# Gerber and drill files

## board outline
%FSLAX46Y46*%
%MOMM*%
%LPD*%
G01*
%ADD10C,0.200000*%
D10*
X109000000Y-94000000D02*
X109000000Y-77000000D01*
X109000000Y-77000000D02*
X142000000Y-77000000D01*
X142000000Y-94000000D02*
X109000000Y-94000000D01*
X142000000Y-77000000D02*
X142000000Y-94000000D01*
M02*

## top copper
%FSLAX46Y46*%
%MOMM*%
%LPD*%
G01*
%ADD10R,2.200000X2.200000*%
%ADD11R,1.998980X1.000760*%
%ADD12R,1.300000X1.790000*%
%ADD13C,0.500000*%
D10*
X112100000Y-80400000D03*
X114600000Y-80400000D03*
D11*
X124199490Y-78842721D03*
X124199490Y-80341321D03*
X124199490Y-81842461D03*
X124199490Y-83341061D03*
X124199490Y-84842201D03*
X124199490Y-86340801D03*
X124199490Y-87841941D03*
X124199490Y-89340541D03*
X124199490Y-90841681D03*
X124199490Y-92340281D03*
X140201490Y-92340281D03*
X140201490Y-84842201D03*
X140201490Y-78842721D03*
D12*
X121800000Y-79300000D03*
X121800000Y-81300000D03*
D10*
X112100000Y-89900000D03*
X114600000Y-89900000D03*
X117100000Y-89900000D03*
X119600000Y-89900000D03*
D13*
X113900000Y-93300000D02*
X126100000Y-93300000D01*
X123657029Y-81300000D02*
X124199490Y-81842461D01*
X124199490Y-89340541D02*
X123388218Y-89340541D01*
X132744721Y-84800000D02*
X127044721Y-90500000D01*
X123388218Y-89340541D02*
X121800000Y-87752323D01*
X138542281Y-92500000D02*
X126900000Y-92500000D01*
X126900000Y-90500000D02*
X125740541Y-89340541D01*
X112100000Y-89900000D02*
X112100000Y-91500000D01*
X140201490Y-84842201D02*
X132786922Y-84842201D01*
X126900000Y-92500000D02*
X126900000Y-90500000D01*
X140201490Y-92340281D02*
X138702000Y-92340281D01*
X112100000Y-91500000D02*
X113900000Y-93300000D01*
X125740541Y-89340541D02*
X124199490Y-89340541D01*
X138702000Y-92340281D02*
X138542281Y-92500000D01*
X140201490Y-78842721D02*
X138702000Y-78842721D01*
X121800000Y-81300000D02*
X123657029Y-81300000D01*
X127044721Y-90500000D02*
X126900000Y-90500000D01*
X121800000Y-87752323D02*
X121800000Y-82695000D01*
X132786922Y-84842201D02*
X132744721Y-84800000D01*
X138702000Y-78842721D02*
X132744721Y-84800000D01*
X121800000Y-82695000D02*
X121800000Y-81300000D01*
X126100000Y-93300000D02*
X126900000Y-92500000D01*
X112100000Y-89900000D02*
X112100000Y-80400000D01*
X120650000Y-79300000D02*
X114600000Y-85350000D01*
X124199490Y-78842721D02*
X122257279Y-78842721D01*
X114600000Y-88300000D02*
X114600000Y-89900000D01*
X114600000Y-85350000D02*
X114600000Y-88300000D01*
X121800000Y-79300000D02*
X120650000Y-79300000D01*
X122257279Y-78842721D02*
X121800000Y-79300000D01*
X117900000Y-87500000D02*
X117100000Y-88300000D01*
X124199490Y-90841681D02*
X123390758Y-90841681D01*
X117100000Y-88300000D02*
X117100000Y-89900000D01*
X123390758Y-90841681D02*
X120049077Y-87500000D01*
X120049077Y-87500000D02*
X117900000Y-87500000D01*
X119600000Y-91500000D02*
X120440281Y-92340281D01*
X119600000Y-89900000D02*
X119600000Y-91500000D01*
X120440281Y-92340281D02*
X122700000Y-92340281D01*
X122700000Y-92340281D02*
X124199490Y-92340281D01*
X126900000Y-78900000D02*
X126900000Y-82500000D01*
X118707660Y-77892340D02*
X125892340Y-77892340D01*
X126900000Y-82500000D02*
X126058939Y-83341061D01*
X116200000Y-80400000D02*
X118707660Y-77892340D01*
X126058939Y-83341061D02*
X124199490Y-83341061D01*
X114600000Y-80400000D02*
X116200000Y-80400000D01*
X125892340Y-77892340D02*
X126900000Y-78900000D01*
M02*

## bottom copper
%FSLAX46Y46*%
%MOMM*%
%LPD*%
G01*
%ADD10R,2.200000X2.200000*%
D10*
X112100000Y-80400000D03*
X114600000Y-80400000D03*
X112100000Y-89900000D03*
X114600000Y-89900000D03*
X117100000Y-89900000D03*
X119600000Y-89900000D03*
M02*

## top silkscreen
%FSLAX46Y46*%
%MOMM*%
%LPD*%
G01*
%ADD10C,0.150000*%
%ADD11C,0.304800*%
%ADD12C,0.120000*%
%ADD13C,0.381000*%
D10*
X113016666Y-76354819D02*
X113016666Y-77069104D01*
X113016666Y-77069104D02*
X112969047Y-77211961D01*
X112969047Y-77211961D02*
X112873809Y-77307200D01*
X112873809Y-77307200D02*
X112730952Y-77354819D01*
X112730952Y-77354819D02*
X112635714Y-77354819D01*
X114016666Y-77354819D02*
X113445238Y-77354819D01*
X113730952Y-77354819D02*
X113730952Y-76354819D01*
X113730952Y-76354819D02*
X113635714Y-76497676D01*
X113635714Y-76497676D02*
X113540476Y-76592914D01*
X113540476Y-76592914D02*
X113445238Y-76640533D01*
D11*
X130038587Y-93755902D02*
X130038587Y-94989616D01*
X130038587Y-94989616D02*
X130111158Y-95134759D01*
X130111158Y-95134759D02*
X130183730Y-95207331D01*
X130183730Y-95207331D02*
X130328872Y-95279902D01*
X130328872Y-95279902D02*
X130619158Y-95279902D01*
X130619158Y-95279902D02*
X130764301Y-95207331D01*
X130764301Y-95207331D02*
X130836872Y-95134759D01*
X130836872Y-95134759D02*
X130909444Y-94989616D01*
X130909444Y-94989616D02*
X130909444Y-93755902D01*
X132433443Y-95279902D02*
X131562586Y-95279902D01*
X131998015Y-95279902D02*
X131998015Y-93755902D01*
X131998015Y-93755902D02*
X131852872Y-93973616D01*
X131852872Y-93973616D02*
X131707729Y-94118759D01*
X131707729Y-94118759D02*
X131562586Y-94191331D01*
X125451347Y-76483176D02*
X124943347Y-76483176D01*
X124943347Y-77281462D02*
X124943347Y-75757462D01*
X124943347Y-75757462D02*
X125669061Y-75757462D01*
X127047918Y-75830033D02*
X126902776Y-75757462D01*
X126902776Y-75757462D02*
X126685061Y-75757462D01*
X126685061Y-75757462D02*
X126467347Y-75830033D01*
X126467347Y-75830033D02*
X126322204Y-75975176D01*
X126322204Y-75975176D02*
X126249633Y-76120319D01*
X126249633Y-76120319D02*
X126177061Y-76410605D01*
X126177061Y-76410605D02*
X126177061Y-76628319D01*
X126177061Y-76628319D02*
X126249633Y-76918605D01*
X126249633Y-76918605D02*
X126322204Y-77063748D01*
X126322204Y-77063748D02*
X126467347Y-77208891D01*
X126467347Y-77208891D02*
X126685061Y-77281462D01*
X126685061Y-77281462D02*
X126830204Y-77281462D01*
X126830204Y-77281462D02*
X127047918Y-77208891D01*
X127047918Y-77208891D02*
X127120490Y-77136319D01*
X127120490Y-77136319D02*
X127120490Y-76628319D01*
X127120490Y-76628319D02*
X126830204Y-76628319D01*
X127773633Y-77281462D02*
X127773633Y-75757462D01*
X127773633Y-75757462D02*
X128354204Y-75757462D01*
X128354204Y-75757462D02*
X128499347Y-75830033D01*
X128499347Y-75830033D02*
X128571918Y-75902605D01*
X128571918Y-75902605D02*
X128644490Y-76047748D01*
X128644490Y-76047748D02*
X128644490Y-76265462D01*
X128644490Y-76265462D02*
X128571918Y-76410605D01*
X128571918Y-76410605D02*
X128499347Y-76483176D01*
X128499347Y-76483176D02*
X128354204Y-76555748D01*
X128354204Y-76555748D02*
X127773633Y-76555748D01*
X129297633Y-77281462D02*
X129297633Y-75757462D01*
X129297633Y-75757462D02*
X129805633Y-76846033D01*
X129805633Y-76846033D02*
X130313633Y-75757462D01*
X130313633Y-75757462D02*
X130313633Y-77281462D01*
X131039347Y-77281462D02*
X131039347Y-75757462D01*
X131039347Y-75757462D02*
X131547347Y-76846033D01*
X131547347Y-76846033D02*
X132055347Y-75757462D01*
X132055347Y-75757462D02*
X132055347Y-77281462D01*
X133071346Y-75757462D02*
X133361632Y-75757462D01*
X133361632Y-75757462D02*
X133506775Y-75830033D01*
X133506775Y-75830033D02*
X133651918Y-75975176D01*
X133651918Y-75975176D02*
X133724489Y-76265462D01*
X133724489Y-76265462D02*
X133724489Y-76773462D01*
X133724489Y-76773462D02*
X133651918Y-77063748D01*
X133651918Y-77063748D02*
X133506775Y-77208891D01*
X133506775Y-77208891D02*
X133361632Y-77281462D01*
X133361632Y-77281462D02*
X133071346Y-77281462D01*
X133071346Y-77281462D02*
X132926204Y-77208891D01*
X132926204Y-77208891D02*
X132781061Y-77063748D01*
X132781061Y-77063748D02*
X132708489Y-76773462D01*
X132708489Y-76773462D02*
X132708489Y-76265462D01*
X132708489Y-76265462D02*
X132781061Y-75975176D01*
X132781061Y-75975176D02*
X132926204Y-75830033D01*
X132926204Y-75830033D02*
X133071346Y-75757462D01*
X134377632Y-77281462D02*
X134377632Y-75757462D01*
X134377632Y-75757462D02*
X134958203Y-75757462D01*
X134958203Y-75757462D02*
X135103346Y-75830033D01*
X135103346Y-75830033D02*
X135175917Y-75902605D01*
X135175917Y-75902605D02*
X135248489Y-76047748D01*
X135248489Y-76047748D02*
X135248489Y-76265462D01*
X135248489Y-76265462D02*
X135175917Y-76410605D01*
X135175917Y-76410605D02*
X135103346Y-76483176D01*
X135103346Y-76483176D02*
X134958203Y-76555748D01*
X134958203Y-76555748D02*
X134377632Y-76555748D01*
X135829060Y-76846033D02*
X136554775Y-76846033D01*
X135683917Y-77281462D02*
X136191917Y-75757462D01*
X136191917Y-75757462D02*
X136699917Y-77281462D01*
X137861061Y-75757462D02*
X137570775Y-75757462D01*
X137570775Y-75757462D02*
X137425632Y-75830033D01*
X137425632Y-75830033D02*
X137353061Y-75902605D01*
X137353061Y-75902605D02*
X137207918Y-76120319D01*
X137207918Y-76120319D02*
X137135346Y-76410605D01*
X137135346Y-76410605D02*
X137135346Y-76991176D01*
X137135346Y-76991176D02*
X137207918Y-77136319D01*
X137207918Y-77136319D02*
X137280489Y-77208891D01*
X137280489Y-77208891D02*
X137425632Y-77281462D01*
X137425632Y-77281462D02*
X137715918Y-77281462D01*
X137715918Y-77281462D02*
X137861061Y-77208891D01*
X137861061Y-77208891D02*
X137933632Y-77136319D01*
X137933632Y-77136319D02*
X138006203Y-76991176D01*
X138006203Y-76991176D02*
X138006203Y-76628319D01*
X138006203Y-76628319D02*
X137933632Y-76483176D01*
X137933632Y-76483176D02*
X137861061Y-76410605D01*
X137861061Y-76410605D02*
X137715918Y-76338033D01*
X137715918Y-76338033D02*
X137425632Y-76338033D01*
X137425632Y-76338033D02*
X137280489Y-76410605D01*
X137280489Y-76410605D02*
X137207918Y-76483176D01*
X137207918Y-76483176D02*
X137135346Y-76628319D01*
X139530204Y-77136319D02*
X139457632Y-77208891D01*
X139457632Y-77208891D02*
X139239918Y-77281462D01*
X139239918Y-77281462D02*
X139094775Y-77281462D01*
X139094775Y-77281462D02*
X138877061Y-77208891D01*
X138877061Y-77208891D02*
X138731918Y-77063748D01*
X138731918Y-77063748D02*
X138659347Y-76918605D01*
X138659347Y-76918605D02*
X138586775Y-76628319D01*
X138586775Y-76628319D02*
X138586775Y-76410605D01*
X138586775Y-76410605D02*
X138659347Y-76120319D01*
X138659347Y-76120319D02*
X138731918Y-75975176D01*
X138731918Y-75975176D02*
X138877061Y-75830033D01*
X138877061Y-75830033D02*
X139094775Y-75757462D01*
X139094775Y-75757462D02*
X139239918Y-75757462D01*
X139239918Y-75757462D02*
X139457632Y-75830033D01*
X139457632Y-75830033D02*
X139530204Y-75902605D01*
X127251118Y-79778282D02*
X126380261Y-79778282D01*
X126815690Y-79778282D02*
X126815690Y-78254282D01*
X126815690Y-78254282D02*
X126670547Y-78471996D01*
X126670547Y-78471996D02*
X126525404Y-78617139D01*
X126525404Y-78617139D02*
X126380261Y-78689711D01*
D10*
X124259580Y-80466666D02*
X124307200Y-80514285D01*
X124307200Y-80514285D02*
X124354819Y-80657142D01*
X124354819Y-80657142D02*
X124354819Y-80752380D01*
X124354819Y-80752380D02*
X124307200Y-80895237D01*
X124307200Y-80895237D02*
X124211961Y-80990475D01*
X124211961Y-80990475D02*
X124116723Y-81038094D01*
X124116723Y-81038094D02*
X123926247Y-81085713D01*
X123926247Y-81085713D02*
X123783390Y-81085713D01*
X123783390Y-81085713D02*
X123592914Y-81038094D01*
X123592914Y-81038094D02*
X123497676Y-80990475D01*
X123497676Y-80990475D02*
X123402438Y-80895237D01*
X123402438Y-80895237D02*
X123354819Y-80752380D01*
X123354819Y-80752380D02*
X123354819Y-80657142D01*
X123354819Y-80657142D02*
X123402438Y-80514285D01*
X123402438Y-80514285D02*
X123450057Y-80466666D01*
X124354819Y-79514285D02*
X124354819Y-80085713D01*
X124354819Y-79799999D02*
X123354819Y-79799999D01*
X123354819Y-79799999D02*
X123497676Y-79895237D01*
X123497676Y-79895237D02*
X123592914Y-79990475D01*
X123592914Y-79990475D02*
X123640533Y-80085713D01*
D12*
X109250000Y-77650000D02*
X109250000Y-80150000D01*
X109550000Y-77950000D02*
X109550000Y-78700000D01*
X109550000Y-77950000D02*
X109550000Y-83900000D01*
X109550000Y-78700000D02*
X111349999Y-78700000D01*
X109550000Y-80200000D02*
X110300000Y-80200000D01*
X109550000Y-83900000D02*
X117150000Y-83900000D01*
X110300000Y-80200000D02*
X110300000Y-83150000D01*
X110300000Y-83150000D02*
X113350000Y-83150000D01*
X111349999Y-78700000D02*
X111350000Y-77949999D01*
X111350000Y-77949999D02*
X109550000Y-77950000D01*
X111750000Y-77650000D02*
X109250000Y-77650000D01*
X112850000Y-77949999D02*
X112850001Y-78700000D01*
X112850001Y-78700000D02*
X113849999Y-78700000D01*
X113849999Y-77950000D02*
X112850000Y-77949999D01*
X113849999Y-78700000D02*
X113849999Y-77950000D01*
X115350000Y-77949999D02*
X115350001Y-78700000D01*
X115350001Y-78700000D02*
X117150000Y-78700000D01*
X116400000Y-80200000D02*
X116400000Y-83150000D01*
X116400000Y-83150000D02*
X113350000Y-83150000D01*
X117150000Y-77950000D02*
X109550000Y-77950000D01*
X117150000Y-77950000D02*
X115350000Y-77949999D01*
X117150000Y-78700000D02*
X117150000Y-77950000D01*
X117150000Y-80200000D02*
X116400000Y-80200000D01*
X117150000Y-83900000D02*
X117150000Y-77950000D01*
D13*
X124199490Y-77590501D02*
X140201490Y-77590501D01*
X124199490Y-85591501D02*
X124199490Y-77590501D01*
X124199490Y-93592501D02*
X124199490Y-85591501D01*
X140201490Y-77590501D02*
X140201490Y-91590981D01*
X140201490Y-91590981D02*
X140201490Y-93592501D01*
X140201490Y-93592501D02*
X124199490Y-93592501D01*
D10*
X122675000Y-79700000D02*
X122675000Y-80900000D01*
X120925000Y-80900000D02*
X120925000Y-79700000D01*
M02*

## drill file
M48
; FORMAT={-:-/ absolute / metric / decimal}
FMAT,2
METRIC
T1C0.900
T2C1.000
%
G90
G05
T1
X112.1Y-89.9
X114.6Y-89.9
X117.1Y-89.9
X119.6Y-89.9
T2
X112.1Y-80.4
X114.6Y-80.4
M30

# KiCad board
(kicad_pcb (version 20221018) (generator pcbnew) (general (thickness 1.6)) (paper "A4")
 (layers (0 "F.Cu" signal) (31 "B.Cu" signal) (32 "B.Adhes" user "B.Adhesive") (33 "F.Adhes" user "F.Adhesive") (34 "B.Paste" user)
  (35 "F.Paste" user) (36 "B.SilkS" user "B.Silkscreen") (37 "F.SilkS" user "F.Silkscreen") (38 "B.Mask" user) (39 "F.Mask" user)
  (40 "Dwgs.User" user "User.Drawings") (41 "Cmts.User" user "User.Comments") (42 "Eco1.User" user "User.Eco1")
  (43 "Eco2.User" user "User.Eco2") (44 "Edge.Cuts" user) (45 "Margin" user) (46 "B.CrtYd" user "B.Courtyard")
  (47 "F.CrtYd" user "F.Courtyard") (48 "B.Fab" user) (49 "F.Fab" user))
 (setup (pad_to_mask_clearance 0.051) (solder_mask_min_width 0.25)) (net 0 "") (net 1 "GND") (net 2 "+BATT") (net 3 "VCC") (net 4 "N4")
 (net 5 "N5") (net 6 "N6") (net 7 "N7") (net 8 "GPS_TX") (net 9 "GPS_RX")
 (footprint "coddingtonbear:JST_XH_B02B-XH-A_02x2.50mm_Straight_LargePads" (layer "F.Cu") (at 112.1 80.4)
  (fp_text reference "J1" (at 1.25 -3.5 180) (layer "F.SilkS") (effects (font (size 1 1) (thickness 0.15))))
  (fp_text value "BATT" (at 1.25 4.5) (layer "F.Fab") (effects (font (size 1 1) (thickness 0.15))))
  (fp_line (start -2.85 -2.75) (end -2.85 -0.25) (stroke (width 0.12) (type solid)) (layer "F.SilkS"))
  (fp_line (start -2.55 -2.45) (end -2.55 -1.7) (stroke (width 0.12) (type solid)) (layer "F.SilkS"))
  (fp_line (start -2.55 -2.45) (end -2.55 3.5) (stroke (width 0.12) (type solid)) (layer "F.SilkS"))
  (fp_line (start -2.55 -1.7) (end -0.750001 -1.7) (stroke (width 0.12) (type solid)) (layer "F.SilkS"))
  (fp_line (start -2.55 -0.2) (end -1.8 -0.2) (stroke (width 0.12) (type solid)) (layer "F.SilkS"))
  (fp_line (start -2.55 3.5) (end 5.05 3.5) (stroke (width 0.12) (type solid)) (layer "F.SilkS"))
  (fp_line (start -1.8 -0.2) (end -1.8 2.75) (stroke (width 0.12) (type solid)) (layer "F.SilkS"))
  (fp_line (start -1.8 2.75) (end 1.25 2.75) (stroke (width 0.12) (type solid)) (layer "F.SilkS"))
  (fp_line (start -0.750001 -1.7) (end -0.75 -2.450001) (stroke (width 0.12) (type solid)) (layer "F.SilkS"))
  (fp_line (start -0.75 -2.450001) (end -2.55 -2.45) (stroke (width 0.12) (type solid)) (layer "F.SilkS"))
  (fp_line (start -0.35 -2.75) (end -2.85 -2.75) (stroke (width 0.12) (type solid)) (layer "F.SilkS"))
  (fp_line (start 0.75 -2.450001) (end 0.750001 -1.7) (stroke (width 0.12) (type solid)) (layer "F.SilkS"))
  (fp_line (start 0.750001 -1.7) (end 1.749999 -1.7) (stroke (width 0.12) (type solid)) (layer "F.SilkS"))
  (fp_line (start 1.749999 -2.45) (end 0.75 -2.450001) (stroke (width 0.12) (type solid)) (layer "F.SilkS"))
  (fp_line (start 1.749999 -1.7) (end 1.749999 -2.45) (stroke (width 0.12) (type solid)) (layer "F.SilkS"))
  (fp_line (start 3.25 -2.450001) (end 3.250001 -1.7) (stroke (width 0.12) (type solid)) (layer "F.SilkS"))
  (fp_line (start 3.250001 -1.7) (end 5.05 -1.7) (stroke (width 0.12) (type solid)) (layer "F.SilkS"))
  (fp_line (start 4.3 -0.2) (end 4.3 2.75) (stroke (width 0.12) (type solid)) (layer "F.SilkS"))
  (fp_line (start 4.3 2.75) (end 1.25 2.75) (stroke (width 0.12) (type solid)) (layer "F.SilkS"))
  (fp_line (start 5.05 -2.45) (end -2.55 -2.45) (stroke (width 0.12) (type solid)) (layer "F.SilkS"))
  (fp_line (start 5.05 -2.45) (end 3.25 -2.450001) (stroke (width 0.12) (type solid)) (layer "F.SilkS"))
  (fp_line (start 5.05 -1.7) (end 5.05 -2.45) (stroke (width 0.12) (type solid)) (layer "F.SilkS"))
  (fp_line (start 5.05 -0.2) (end 4.3 -0.2) (stroke (width 0.12) (type solid)) (layer "F.SilkS"))
  (fp_line (start 5.05 3.5) (end 5.05 -2.45) (stroke (width 0.12) (type solid)) (layer "F.SilkS"))
  (pad "1" thru_hole rect (at 0 0) (size 2.2 2.2) (drill 1) (layers "*.Cu" "*.Mask") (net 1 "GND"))
  (pad "2" thru_hole rect (at 2.5 0) (size 2.2 2.2) (drill 1) (layers "*.Cu" "*.Mask") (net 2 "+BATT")))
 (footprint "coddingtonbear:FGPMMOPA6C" (layer "F.Cu") (at 132.20049 85.591501)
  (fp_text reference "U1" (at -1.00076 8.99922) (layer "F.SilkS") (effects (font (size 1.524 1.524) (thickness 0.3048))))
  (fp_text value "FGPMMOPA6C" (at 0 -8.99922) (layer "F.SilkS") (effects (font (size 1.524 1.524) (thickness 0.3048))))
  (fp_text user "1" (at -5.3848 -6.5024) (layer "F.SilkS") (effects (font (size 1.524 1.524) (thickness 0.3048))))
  (fp_line (start -8.001 -8.001) (end 8.001 -8.001) (stroke (width 0.381) (type solid)) (layer "F.SilkS"))
  (fp_line (start -8.001 0) (end -8.001 -8.001) (stroke (width 0.381) (type solid)) (layer "F.SilkS"))
  (fp_line (start -8.001 8.001) (end -8.001 0) (stroke (width 0.381) (type solid)) (layer "F.SilkS"))
  (fp_line (start 8.001 -8.001) (end 8.001 5.99948) (stroke (width 0.381) (type solid)) (layer "F.SilkS"))
  (fp_line (start 8.001 5.99948) (end 8.001 8.001) (stroke (width 0.381) (type solid)) (layer "F.SilkS"))
  (fp_line (start 8.001 8.001) (end -8.001 8.001) (stroke (width 0.381) (type solid)) (layer "F.SilkS"))
  (pad "1" smd rect (at -8.001 -6.74878) (size 1.99898 1.00076) (layers "F.Cu" "F.Paste" "F.Mask") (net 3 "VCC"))
  (pad "2" smd rect (at -8.001 -5.25018) (size 1.99898 1.00076) (layers "F.Cu" "F.Paste" "F.Mask") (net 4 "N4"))
  (pad "3" smd rect (at -8.001 -3.74904) (size 1.99898 1.00076) (layers "F.Cu" "F.Paste" "F.Mask") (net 1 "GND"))
  (pad "4" smd rect (at -8.001 -2.25044) (size 1.99898 1.00076) (layers "F.Cu" "F.Paste" "F.Mask") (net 2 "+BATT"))
  (pad "5" smd rect (at -8.001 -0.7493) (size 1.99898 1.00076) (layers "F.Cu" "F.Paste" "F.Mask") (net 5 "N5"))
  (pad "6" smd rect (at -8.001 0.7493) (size 1.99898 1.00076) (layers "F.Cu" "F.Paste" "F.Mask") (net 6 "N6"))
  (pad "7" smd rect (at -8.001 2.25044) (size 1.99898 1.00076) (layers "F.Cu" "F.Paste" "F.Mask") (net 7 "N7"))
  (pad "8" smd rect (at -8.001 3.74904) (size 1.99898 1.00076) (layers "F.Cu" "F.Paste" "F.Mask") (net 1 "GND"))
  (pad "9" smd rect (at -8.001 5.25018) (size 1.99898 1.00076) (layers "F.Cu" "F.Paste" "F.Mask") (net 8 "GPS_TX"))
  (pad "10" smd rect (at -8.001 6.74878) (size 1.99898 1.00076) (layers "F.Cu" "F.Paste" "F.Mask") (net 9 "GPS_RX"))
  (pad "11" smd rect (at 8.001 6.74878) (size 1.99898 1.00076) (layers "F.Cu" "F.Paste" "F.Mask") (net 1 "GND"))
  (pad "12" smd rect (at 8.001 -0.7493) (size 1.99898 1.00076) (layers "F.Cu" "F.Paste" "F.Mask") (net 1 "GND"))
  (pad "13" smd rect (at 8.001 -6.74878) (size 1.99898 1.00076) (layers "F.Cu" "F.Paste" "F.Mask") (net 1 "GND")))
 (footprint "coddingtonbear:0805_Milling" (layer "F.Cu") (at 121.8 80.3 -90)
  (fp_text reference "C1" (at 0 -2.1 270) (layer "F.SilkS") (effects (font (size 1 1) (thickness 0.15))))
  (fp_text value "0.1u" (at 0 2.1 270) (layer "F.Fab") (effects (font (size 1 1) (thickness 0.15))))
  (fp_line (start -0.6 -0.875) (end 0.6 -0.875) (stroke (width 0.15) (type solid)) (layer "F.SilkS"))
  (fp_line (start 0.6 0.875) (end -0.6 0.875) (stroke (width 0.15) (type solid)) (layer "F.SilkS"))
  (pad "1" smd rect (at -1 0 270) (size 1.79 1.3) (layers "F.Cu" "F.Paste" "F.Mask") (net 3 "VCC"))
  (pad "2" smd rect (at 1 0 270) (size 1.79 1.3) (layers "F.Cu" "F.Paste" "F.Mask") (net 1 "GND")))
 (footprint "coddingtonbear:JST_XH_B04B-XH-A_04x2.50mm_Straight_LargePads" (layer "B.Cu") (at 112.1 89.9)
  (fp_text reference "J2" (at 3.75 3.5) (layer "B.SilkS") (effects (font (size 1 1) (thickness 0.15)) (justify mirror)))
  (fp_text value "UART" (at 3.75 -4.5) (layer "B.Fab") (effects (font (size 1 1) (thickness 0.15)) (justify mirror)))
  (pad "1" thru_hole rect (at 0 0) (size 2.2 2.2) (drill 0.9) (layers "*.Cu" "*.Mask") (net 1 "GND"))
  (pad "2" thru_hole rect (at 2.5 0) (size 2.2 2.2) (drill 0.9) (layers "*.Cu" "*.Mask") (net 3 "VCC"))
  (pad "3" thru_hole rect (at 5 0) (size 2.2 2.2) (drill 0.9) (layers "*.Cu" "*.Mask") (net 8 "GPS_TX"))
  (pad "4" thru_hole rect (at 7.5 0) (size 2.2 2.2) (drill 0.9) (layers "*.Cu" "*.Mask") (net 9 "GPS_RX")))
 (gr_line (start 109 94) (end 109 77) (stroke (width 0.2) (type solid)) (layer "Edge.Cuts"))
 (gr_line (start 109 77) (end 142 77) (stroke (width 0.2) (type solid)) (layer "Edge.Cuts"))
 (gr_line (start 142 94) (end 109 94) (stroke (width 0.2) (type solid)) (layer "Edge.Cuts"))
 (gr_line (start 142 77) (end 142 94) (stroke (width 0.2) (type solid)) (layer "Edge.Cuts"))
 (segment (start 113.9 93.3) (end 126.1 93.3) (width 0.5) (layer "F.Cu") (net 1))
 (segment (start 123.657029 81.3) (end 124.19949 81.842461) (width 0.5) (layer "F.Cu") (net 1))
 (segment (start 124.19949 89.340541) (end 123.388218 89.340541) (width 0.5) (layer "F.Cu") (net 1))
 (segment (start 132.744721 84.8) (end 127.044721 90.5) (width 0.5) (layer "F.Cu") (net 1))
 (segment (start 123.388218 89.340541) (end 121.8 87.752323) (width 0.5) (layer "F.Cu") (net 1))
 (segment (start 138.542281 92.5) (end 126.9 92.5) (width 0.5) (layer "F.Cu") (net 1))
 (segment (start 126.9 90.5) (end 125.740541 89.340541) (width 0.5) (layer "F.Cu") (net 1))
 (segment (start 112.1 89.9) (end 112.1 91.5) (width 0.5) (layer "F.Cu") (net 1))
 (segment (start 140.20149 84.842201) (end 132.786922 84.842201) (width 0.5) (layer "F.Cu") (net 1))
 (segment (start 126.9 92.5) (end 126.9 90.5) (width 0.5) (layer "F.Cu") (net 1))
 (segment (start 140.20149 92.340281) (end 138.702 92.340281) (width 0.5) (layer "F.Cu") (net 1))
 (segment (start 112.1 91.5) (end 113.9 93.3) (width 0.5) (layer "F.Cu") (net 1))
 (segment (start 125.740541 89.340541) (end 124.19949 89.340541) (width 0.5) (layer "F.Cu") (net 1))
 (segment (start 138.702 92.340281) (end 138.542281 92.5) (width 0.5) (layer "F.Cu") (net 1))
 (segment (start 140.20149 78.842721) (end 138.702 78.842721) (width 0.5) (layer "F.Cu") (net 1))
 (segment (start 121.8 81.3) (end 123.657029 81.3) (width 0.5) (layer "F.Cu") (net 1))
 (segment (start 127.044721 90.5) (end 126.9 90.5) (width 0.5) (layer "F.Cu") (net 1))
 (segment (start 121.8 87.752323) (end 121.8 82.695) (width 0.5) (layer "F.Cu") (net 1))
 (segment (start 132.786922 84.842201) (end 132.744721 84.8) (width 0.5) (layer "F.Cu") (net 1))
 (segment (start 138.702 78.842721) (end 132.744721 84.8) (width 0.5) (layer "F.Cu") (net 1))
 (segment (start 121.8 82.695) (end 121.8 81.3) (width 0.5) (layer "F.Cu") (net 1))
 (segment (start 126.1 93.3) (end 126.9 92.5) (width 0.5) (layer "F.Cu") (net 1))
 (segment (start 112.1 89.9) (end 112.1 80.4) (width 0.5) (layer "F.Cu") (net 1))
 (segment (start 120.65 79.3) (end 114.6 85.35) (width 0.5) (layer "F.Cu") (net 3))
 (segment (start 124.19949 78.842721) (end 122.257279 78.842721) (width 0.5) (layer "F.Cu") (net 3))
 (segment (start 114.6 88.3) (end 114.6 89.9) (width 0.5) (layer "F.Cu") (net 3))
 (segment (start 114.6 85.35) (end 114.6 88.3) (width 0.5) (layer "F.Cu") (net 3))
 (segment (start 121.8 79.3) (end 120.65 79.3) (width 0.5) (layer "F.Cu") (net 3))
 (segment (start 122.257279 78.842721) (end 121.8 79.3) (width 0.5) (layer "F.Cu") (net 3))
 (segment (start 117.9 87.5) (end 117.1 88.3) (width 0.5) (layer "F.Cu") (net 8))
 (segment (start 124.19949 90.841681) (end 123.390758 90.841681) (width 0.5) (layer "F.Cu") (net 8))
 (segment (start 117.1 88.3) (end 117.1 89.9) (width 0.5) (layer "F.Cu") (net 8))
 (segment (start 123.390758 90.841681) (end 120.049077 87.5) (width 0.5) (layer "F.Cu") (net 8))
 (segment (start 120.049077 87.5) (end 117.9 87.5) (width 0.5) (layer "F.Cu") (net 8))
 (segment (start 119.6 91.5) (end 120.440281 92.340281) (width 0.5) (layer "F.Cu") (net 9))
 (segment (start 119.6 89.9) (end 119.6 91.5) (width 0.5) (layer "F.Cu") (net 9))
 (segment (start 120.440281 92.340281) (end 122.7 92.340281) (width 0.5) (layer "F.Cu") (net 9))
 (segment (start 122.7 92.340281) (end 124.19949 92.340281) (width 0.5) (layer "F.Cu") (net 9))
 (segment (start 126.9 78.9) (end 126.9 82.5) (width 0.5) (layer "F.Cu") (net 2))
 (segment (start 118.70766 77.89234) (end 125.89234 77.89234) (width 0.5) (layer "F.Cu") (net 2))
 (segment (start 126.9 82.5) (end 126.058939 83.341061) (width 0.5) (layer "F.Cu") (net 2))
 (segment (start 116.2 80.4) (end 118.70766 77.89234) (width 0.5) (layer "F.Cu") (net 2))
 (segment (start 126.058939 83.341061) (end 124.19949 83.341061) (width 0.5) (layer "F.Cu") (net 2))
 (segment (start 114.6 80.4) (end 116.2 80.4) (width 0.5) (layer "F.Cu") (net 2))
 (segment (start 125.89234 77.89234) (end 126.9 78.9) (width 0.5) (layer "F.Cu") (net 2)))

